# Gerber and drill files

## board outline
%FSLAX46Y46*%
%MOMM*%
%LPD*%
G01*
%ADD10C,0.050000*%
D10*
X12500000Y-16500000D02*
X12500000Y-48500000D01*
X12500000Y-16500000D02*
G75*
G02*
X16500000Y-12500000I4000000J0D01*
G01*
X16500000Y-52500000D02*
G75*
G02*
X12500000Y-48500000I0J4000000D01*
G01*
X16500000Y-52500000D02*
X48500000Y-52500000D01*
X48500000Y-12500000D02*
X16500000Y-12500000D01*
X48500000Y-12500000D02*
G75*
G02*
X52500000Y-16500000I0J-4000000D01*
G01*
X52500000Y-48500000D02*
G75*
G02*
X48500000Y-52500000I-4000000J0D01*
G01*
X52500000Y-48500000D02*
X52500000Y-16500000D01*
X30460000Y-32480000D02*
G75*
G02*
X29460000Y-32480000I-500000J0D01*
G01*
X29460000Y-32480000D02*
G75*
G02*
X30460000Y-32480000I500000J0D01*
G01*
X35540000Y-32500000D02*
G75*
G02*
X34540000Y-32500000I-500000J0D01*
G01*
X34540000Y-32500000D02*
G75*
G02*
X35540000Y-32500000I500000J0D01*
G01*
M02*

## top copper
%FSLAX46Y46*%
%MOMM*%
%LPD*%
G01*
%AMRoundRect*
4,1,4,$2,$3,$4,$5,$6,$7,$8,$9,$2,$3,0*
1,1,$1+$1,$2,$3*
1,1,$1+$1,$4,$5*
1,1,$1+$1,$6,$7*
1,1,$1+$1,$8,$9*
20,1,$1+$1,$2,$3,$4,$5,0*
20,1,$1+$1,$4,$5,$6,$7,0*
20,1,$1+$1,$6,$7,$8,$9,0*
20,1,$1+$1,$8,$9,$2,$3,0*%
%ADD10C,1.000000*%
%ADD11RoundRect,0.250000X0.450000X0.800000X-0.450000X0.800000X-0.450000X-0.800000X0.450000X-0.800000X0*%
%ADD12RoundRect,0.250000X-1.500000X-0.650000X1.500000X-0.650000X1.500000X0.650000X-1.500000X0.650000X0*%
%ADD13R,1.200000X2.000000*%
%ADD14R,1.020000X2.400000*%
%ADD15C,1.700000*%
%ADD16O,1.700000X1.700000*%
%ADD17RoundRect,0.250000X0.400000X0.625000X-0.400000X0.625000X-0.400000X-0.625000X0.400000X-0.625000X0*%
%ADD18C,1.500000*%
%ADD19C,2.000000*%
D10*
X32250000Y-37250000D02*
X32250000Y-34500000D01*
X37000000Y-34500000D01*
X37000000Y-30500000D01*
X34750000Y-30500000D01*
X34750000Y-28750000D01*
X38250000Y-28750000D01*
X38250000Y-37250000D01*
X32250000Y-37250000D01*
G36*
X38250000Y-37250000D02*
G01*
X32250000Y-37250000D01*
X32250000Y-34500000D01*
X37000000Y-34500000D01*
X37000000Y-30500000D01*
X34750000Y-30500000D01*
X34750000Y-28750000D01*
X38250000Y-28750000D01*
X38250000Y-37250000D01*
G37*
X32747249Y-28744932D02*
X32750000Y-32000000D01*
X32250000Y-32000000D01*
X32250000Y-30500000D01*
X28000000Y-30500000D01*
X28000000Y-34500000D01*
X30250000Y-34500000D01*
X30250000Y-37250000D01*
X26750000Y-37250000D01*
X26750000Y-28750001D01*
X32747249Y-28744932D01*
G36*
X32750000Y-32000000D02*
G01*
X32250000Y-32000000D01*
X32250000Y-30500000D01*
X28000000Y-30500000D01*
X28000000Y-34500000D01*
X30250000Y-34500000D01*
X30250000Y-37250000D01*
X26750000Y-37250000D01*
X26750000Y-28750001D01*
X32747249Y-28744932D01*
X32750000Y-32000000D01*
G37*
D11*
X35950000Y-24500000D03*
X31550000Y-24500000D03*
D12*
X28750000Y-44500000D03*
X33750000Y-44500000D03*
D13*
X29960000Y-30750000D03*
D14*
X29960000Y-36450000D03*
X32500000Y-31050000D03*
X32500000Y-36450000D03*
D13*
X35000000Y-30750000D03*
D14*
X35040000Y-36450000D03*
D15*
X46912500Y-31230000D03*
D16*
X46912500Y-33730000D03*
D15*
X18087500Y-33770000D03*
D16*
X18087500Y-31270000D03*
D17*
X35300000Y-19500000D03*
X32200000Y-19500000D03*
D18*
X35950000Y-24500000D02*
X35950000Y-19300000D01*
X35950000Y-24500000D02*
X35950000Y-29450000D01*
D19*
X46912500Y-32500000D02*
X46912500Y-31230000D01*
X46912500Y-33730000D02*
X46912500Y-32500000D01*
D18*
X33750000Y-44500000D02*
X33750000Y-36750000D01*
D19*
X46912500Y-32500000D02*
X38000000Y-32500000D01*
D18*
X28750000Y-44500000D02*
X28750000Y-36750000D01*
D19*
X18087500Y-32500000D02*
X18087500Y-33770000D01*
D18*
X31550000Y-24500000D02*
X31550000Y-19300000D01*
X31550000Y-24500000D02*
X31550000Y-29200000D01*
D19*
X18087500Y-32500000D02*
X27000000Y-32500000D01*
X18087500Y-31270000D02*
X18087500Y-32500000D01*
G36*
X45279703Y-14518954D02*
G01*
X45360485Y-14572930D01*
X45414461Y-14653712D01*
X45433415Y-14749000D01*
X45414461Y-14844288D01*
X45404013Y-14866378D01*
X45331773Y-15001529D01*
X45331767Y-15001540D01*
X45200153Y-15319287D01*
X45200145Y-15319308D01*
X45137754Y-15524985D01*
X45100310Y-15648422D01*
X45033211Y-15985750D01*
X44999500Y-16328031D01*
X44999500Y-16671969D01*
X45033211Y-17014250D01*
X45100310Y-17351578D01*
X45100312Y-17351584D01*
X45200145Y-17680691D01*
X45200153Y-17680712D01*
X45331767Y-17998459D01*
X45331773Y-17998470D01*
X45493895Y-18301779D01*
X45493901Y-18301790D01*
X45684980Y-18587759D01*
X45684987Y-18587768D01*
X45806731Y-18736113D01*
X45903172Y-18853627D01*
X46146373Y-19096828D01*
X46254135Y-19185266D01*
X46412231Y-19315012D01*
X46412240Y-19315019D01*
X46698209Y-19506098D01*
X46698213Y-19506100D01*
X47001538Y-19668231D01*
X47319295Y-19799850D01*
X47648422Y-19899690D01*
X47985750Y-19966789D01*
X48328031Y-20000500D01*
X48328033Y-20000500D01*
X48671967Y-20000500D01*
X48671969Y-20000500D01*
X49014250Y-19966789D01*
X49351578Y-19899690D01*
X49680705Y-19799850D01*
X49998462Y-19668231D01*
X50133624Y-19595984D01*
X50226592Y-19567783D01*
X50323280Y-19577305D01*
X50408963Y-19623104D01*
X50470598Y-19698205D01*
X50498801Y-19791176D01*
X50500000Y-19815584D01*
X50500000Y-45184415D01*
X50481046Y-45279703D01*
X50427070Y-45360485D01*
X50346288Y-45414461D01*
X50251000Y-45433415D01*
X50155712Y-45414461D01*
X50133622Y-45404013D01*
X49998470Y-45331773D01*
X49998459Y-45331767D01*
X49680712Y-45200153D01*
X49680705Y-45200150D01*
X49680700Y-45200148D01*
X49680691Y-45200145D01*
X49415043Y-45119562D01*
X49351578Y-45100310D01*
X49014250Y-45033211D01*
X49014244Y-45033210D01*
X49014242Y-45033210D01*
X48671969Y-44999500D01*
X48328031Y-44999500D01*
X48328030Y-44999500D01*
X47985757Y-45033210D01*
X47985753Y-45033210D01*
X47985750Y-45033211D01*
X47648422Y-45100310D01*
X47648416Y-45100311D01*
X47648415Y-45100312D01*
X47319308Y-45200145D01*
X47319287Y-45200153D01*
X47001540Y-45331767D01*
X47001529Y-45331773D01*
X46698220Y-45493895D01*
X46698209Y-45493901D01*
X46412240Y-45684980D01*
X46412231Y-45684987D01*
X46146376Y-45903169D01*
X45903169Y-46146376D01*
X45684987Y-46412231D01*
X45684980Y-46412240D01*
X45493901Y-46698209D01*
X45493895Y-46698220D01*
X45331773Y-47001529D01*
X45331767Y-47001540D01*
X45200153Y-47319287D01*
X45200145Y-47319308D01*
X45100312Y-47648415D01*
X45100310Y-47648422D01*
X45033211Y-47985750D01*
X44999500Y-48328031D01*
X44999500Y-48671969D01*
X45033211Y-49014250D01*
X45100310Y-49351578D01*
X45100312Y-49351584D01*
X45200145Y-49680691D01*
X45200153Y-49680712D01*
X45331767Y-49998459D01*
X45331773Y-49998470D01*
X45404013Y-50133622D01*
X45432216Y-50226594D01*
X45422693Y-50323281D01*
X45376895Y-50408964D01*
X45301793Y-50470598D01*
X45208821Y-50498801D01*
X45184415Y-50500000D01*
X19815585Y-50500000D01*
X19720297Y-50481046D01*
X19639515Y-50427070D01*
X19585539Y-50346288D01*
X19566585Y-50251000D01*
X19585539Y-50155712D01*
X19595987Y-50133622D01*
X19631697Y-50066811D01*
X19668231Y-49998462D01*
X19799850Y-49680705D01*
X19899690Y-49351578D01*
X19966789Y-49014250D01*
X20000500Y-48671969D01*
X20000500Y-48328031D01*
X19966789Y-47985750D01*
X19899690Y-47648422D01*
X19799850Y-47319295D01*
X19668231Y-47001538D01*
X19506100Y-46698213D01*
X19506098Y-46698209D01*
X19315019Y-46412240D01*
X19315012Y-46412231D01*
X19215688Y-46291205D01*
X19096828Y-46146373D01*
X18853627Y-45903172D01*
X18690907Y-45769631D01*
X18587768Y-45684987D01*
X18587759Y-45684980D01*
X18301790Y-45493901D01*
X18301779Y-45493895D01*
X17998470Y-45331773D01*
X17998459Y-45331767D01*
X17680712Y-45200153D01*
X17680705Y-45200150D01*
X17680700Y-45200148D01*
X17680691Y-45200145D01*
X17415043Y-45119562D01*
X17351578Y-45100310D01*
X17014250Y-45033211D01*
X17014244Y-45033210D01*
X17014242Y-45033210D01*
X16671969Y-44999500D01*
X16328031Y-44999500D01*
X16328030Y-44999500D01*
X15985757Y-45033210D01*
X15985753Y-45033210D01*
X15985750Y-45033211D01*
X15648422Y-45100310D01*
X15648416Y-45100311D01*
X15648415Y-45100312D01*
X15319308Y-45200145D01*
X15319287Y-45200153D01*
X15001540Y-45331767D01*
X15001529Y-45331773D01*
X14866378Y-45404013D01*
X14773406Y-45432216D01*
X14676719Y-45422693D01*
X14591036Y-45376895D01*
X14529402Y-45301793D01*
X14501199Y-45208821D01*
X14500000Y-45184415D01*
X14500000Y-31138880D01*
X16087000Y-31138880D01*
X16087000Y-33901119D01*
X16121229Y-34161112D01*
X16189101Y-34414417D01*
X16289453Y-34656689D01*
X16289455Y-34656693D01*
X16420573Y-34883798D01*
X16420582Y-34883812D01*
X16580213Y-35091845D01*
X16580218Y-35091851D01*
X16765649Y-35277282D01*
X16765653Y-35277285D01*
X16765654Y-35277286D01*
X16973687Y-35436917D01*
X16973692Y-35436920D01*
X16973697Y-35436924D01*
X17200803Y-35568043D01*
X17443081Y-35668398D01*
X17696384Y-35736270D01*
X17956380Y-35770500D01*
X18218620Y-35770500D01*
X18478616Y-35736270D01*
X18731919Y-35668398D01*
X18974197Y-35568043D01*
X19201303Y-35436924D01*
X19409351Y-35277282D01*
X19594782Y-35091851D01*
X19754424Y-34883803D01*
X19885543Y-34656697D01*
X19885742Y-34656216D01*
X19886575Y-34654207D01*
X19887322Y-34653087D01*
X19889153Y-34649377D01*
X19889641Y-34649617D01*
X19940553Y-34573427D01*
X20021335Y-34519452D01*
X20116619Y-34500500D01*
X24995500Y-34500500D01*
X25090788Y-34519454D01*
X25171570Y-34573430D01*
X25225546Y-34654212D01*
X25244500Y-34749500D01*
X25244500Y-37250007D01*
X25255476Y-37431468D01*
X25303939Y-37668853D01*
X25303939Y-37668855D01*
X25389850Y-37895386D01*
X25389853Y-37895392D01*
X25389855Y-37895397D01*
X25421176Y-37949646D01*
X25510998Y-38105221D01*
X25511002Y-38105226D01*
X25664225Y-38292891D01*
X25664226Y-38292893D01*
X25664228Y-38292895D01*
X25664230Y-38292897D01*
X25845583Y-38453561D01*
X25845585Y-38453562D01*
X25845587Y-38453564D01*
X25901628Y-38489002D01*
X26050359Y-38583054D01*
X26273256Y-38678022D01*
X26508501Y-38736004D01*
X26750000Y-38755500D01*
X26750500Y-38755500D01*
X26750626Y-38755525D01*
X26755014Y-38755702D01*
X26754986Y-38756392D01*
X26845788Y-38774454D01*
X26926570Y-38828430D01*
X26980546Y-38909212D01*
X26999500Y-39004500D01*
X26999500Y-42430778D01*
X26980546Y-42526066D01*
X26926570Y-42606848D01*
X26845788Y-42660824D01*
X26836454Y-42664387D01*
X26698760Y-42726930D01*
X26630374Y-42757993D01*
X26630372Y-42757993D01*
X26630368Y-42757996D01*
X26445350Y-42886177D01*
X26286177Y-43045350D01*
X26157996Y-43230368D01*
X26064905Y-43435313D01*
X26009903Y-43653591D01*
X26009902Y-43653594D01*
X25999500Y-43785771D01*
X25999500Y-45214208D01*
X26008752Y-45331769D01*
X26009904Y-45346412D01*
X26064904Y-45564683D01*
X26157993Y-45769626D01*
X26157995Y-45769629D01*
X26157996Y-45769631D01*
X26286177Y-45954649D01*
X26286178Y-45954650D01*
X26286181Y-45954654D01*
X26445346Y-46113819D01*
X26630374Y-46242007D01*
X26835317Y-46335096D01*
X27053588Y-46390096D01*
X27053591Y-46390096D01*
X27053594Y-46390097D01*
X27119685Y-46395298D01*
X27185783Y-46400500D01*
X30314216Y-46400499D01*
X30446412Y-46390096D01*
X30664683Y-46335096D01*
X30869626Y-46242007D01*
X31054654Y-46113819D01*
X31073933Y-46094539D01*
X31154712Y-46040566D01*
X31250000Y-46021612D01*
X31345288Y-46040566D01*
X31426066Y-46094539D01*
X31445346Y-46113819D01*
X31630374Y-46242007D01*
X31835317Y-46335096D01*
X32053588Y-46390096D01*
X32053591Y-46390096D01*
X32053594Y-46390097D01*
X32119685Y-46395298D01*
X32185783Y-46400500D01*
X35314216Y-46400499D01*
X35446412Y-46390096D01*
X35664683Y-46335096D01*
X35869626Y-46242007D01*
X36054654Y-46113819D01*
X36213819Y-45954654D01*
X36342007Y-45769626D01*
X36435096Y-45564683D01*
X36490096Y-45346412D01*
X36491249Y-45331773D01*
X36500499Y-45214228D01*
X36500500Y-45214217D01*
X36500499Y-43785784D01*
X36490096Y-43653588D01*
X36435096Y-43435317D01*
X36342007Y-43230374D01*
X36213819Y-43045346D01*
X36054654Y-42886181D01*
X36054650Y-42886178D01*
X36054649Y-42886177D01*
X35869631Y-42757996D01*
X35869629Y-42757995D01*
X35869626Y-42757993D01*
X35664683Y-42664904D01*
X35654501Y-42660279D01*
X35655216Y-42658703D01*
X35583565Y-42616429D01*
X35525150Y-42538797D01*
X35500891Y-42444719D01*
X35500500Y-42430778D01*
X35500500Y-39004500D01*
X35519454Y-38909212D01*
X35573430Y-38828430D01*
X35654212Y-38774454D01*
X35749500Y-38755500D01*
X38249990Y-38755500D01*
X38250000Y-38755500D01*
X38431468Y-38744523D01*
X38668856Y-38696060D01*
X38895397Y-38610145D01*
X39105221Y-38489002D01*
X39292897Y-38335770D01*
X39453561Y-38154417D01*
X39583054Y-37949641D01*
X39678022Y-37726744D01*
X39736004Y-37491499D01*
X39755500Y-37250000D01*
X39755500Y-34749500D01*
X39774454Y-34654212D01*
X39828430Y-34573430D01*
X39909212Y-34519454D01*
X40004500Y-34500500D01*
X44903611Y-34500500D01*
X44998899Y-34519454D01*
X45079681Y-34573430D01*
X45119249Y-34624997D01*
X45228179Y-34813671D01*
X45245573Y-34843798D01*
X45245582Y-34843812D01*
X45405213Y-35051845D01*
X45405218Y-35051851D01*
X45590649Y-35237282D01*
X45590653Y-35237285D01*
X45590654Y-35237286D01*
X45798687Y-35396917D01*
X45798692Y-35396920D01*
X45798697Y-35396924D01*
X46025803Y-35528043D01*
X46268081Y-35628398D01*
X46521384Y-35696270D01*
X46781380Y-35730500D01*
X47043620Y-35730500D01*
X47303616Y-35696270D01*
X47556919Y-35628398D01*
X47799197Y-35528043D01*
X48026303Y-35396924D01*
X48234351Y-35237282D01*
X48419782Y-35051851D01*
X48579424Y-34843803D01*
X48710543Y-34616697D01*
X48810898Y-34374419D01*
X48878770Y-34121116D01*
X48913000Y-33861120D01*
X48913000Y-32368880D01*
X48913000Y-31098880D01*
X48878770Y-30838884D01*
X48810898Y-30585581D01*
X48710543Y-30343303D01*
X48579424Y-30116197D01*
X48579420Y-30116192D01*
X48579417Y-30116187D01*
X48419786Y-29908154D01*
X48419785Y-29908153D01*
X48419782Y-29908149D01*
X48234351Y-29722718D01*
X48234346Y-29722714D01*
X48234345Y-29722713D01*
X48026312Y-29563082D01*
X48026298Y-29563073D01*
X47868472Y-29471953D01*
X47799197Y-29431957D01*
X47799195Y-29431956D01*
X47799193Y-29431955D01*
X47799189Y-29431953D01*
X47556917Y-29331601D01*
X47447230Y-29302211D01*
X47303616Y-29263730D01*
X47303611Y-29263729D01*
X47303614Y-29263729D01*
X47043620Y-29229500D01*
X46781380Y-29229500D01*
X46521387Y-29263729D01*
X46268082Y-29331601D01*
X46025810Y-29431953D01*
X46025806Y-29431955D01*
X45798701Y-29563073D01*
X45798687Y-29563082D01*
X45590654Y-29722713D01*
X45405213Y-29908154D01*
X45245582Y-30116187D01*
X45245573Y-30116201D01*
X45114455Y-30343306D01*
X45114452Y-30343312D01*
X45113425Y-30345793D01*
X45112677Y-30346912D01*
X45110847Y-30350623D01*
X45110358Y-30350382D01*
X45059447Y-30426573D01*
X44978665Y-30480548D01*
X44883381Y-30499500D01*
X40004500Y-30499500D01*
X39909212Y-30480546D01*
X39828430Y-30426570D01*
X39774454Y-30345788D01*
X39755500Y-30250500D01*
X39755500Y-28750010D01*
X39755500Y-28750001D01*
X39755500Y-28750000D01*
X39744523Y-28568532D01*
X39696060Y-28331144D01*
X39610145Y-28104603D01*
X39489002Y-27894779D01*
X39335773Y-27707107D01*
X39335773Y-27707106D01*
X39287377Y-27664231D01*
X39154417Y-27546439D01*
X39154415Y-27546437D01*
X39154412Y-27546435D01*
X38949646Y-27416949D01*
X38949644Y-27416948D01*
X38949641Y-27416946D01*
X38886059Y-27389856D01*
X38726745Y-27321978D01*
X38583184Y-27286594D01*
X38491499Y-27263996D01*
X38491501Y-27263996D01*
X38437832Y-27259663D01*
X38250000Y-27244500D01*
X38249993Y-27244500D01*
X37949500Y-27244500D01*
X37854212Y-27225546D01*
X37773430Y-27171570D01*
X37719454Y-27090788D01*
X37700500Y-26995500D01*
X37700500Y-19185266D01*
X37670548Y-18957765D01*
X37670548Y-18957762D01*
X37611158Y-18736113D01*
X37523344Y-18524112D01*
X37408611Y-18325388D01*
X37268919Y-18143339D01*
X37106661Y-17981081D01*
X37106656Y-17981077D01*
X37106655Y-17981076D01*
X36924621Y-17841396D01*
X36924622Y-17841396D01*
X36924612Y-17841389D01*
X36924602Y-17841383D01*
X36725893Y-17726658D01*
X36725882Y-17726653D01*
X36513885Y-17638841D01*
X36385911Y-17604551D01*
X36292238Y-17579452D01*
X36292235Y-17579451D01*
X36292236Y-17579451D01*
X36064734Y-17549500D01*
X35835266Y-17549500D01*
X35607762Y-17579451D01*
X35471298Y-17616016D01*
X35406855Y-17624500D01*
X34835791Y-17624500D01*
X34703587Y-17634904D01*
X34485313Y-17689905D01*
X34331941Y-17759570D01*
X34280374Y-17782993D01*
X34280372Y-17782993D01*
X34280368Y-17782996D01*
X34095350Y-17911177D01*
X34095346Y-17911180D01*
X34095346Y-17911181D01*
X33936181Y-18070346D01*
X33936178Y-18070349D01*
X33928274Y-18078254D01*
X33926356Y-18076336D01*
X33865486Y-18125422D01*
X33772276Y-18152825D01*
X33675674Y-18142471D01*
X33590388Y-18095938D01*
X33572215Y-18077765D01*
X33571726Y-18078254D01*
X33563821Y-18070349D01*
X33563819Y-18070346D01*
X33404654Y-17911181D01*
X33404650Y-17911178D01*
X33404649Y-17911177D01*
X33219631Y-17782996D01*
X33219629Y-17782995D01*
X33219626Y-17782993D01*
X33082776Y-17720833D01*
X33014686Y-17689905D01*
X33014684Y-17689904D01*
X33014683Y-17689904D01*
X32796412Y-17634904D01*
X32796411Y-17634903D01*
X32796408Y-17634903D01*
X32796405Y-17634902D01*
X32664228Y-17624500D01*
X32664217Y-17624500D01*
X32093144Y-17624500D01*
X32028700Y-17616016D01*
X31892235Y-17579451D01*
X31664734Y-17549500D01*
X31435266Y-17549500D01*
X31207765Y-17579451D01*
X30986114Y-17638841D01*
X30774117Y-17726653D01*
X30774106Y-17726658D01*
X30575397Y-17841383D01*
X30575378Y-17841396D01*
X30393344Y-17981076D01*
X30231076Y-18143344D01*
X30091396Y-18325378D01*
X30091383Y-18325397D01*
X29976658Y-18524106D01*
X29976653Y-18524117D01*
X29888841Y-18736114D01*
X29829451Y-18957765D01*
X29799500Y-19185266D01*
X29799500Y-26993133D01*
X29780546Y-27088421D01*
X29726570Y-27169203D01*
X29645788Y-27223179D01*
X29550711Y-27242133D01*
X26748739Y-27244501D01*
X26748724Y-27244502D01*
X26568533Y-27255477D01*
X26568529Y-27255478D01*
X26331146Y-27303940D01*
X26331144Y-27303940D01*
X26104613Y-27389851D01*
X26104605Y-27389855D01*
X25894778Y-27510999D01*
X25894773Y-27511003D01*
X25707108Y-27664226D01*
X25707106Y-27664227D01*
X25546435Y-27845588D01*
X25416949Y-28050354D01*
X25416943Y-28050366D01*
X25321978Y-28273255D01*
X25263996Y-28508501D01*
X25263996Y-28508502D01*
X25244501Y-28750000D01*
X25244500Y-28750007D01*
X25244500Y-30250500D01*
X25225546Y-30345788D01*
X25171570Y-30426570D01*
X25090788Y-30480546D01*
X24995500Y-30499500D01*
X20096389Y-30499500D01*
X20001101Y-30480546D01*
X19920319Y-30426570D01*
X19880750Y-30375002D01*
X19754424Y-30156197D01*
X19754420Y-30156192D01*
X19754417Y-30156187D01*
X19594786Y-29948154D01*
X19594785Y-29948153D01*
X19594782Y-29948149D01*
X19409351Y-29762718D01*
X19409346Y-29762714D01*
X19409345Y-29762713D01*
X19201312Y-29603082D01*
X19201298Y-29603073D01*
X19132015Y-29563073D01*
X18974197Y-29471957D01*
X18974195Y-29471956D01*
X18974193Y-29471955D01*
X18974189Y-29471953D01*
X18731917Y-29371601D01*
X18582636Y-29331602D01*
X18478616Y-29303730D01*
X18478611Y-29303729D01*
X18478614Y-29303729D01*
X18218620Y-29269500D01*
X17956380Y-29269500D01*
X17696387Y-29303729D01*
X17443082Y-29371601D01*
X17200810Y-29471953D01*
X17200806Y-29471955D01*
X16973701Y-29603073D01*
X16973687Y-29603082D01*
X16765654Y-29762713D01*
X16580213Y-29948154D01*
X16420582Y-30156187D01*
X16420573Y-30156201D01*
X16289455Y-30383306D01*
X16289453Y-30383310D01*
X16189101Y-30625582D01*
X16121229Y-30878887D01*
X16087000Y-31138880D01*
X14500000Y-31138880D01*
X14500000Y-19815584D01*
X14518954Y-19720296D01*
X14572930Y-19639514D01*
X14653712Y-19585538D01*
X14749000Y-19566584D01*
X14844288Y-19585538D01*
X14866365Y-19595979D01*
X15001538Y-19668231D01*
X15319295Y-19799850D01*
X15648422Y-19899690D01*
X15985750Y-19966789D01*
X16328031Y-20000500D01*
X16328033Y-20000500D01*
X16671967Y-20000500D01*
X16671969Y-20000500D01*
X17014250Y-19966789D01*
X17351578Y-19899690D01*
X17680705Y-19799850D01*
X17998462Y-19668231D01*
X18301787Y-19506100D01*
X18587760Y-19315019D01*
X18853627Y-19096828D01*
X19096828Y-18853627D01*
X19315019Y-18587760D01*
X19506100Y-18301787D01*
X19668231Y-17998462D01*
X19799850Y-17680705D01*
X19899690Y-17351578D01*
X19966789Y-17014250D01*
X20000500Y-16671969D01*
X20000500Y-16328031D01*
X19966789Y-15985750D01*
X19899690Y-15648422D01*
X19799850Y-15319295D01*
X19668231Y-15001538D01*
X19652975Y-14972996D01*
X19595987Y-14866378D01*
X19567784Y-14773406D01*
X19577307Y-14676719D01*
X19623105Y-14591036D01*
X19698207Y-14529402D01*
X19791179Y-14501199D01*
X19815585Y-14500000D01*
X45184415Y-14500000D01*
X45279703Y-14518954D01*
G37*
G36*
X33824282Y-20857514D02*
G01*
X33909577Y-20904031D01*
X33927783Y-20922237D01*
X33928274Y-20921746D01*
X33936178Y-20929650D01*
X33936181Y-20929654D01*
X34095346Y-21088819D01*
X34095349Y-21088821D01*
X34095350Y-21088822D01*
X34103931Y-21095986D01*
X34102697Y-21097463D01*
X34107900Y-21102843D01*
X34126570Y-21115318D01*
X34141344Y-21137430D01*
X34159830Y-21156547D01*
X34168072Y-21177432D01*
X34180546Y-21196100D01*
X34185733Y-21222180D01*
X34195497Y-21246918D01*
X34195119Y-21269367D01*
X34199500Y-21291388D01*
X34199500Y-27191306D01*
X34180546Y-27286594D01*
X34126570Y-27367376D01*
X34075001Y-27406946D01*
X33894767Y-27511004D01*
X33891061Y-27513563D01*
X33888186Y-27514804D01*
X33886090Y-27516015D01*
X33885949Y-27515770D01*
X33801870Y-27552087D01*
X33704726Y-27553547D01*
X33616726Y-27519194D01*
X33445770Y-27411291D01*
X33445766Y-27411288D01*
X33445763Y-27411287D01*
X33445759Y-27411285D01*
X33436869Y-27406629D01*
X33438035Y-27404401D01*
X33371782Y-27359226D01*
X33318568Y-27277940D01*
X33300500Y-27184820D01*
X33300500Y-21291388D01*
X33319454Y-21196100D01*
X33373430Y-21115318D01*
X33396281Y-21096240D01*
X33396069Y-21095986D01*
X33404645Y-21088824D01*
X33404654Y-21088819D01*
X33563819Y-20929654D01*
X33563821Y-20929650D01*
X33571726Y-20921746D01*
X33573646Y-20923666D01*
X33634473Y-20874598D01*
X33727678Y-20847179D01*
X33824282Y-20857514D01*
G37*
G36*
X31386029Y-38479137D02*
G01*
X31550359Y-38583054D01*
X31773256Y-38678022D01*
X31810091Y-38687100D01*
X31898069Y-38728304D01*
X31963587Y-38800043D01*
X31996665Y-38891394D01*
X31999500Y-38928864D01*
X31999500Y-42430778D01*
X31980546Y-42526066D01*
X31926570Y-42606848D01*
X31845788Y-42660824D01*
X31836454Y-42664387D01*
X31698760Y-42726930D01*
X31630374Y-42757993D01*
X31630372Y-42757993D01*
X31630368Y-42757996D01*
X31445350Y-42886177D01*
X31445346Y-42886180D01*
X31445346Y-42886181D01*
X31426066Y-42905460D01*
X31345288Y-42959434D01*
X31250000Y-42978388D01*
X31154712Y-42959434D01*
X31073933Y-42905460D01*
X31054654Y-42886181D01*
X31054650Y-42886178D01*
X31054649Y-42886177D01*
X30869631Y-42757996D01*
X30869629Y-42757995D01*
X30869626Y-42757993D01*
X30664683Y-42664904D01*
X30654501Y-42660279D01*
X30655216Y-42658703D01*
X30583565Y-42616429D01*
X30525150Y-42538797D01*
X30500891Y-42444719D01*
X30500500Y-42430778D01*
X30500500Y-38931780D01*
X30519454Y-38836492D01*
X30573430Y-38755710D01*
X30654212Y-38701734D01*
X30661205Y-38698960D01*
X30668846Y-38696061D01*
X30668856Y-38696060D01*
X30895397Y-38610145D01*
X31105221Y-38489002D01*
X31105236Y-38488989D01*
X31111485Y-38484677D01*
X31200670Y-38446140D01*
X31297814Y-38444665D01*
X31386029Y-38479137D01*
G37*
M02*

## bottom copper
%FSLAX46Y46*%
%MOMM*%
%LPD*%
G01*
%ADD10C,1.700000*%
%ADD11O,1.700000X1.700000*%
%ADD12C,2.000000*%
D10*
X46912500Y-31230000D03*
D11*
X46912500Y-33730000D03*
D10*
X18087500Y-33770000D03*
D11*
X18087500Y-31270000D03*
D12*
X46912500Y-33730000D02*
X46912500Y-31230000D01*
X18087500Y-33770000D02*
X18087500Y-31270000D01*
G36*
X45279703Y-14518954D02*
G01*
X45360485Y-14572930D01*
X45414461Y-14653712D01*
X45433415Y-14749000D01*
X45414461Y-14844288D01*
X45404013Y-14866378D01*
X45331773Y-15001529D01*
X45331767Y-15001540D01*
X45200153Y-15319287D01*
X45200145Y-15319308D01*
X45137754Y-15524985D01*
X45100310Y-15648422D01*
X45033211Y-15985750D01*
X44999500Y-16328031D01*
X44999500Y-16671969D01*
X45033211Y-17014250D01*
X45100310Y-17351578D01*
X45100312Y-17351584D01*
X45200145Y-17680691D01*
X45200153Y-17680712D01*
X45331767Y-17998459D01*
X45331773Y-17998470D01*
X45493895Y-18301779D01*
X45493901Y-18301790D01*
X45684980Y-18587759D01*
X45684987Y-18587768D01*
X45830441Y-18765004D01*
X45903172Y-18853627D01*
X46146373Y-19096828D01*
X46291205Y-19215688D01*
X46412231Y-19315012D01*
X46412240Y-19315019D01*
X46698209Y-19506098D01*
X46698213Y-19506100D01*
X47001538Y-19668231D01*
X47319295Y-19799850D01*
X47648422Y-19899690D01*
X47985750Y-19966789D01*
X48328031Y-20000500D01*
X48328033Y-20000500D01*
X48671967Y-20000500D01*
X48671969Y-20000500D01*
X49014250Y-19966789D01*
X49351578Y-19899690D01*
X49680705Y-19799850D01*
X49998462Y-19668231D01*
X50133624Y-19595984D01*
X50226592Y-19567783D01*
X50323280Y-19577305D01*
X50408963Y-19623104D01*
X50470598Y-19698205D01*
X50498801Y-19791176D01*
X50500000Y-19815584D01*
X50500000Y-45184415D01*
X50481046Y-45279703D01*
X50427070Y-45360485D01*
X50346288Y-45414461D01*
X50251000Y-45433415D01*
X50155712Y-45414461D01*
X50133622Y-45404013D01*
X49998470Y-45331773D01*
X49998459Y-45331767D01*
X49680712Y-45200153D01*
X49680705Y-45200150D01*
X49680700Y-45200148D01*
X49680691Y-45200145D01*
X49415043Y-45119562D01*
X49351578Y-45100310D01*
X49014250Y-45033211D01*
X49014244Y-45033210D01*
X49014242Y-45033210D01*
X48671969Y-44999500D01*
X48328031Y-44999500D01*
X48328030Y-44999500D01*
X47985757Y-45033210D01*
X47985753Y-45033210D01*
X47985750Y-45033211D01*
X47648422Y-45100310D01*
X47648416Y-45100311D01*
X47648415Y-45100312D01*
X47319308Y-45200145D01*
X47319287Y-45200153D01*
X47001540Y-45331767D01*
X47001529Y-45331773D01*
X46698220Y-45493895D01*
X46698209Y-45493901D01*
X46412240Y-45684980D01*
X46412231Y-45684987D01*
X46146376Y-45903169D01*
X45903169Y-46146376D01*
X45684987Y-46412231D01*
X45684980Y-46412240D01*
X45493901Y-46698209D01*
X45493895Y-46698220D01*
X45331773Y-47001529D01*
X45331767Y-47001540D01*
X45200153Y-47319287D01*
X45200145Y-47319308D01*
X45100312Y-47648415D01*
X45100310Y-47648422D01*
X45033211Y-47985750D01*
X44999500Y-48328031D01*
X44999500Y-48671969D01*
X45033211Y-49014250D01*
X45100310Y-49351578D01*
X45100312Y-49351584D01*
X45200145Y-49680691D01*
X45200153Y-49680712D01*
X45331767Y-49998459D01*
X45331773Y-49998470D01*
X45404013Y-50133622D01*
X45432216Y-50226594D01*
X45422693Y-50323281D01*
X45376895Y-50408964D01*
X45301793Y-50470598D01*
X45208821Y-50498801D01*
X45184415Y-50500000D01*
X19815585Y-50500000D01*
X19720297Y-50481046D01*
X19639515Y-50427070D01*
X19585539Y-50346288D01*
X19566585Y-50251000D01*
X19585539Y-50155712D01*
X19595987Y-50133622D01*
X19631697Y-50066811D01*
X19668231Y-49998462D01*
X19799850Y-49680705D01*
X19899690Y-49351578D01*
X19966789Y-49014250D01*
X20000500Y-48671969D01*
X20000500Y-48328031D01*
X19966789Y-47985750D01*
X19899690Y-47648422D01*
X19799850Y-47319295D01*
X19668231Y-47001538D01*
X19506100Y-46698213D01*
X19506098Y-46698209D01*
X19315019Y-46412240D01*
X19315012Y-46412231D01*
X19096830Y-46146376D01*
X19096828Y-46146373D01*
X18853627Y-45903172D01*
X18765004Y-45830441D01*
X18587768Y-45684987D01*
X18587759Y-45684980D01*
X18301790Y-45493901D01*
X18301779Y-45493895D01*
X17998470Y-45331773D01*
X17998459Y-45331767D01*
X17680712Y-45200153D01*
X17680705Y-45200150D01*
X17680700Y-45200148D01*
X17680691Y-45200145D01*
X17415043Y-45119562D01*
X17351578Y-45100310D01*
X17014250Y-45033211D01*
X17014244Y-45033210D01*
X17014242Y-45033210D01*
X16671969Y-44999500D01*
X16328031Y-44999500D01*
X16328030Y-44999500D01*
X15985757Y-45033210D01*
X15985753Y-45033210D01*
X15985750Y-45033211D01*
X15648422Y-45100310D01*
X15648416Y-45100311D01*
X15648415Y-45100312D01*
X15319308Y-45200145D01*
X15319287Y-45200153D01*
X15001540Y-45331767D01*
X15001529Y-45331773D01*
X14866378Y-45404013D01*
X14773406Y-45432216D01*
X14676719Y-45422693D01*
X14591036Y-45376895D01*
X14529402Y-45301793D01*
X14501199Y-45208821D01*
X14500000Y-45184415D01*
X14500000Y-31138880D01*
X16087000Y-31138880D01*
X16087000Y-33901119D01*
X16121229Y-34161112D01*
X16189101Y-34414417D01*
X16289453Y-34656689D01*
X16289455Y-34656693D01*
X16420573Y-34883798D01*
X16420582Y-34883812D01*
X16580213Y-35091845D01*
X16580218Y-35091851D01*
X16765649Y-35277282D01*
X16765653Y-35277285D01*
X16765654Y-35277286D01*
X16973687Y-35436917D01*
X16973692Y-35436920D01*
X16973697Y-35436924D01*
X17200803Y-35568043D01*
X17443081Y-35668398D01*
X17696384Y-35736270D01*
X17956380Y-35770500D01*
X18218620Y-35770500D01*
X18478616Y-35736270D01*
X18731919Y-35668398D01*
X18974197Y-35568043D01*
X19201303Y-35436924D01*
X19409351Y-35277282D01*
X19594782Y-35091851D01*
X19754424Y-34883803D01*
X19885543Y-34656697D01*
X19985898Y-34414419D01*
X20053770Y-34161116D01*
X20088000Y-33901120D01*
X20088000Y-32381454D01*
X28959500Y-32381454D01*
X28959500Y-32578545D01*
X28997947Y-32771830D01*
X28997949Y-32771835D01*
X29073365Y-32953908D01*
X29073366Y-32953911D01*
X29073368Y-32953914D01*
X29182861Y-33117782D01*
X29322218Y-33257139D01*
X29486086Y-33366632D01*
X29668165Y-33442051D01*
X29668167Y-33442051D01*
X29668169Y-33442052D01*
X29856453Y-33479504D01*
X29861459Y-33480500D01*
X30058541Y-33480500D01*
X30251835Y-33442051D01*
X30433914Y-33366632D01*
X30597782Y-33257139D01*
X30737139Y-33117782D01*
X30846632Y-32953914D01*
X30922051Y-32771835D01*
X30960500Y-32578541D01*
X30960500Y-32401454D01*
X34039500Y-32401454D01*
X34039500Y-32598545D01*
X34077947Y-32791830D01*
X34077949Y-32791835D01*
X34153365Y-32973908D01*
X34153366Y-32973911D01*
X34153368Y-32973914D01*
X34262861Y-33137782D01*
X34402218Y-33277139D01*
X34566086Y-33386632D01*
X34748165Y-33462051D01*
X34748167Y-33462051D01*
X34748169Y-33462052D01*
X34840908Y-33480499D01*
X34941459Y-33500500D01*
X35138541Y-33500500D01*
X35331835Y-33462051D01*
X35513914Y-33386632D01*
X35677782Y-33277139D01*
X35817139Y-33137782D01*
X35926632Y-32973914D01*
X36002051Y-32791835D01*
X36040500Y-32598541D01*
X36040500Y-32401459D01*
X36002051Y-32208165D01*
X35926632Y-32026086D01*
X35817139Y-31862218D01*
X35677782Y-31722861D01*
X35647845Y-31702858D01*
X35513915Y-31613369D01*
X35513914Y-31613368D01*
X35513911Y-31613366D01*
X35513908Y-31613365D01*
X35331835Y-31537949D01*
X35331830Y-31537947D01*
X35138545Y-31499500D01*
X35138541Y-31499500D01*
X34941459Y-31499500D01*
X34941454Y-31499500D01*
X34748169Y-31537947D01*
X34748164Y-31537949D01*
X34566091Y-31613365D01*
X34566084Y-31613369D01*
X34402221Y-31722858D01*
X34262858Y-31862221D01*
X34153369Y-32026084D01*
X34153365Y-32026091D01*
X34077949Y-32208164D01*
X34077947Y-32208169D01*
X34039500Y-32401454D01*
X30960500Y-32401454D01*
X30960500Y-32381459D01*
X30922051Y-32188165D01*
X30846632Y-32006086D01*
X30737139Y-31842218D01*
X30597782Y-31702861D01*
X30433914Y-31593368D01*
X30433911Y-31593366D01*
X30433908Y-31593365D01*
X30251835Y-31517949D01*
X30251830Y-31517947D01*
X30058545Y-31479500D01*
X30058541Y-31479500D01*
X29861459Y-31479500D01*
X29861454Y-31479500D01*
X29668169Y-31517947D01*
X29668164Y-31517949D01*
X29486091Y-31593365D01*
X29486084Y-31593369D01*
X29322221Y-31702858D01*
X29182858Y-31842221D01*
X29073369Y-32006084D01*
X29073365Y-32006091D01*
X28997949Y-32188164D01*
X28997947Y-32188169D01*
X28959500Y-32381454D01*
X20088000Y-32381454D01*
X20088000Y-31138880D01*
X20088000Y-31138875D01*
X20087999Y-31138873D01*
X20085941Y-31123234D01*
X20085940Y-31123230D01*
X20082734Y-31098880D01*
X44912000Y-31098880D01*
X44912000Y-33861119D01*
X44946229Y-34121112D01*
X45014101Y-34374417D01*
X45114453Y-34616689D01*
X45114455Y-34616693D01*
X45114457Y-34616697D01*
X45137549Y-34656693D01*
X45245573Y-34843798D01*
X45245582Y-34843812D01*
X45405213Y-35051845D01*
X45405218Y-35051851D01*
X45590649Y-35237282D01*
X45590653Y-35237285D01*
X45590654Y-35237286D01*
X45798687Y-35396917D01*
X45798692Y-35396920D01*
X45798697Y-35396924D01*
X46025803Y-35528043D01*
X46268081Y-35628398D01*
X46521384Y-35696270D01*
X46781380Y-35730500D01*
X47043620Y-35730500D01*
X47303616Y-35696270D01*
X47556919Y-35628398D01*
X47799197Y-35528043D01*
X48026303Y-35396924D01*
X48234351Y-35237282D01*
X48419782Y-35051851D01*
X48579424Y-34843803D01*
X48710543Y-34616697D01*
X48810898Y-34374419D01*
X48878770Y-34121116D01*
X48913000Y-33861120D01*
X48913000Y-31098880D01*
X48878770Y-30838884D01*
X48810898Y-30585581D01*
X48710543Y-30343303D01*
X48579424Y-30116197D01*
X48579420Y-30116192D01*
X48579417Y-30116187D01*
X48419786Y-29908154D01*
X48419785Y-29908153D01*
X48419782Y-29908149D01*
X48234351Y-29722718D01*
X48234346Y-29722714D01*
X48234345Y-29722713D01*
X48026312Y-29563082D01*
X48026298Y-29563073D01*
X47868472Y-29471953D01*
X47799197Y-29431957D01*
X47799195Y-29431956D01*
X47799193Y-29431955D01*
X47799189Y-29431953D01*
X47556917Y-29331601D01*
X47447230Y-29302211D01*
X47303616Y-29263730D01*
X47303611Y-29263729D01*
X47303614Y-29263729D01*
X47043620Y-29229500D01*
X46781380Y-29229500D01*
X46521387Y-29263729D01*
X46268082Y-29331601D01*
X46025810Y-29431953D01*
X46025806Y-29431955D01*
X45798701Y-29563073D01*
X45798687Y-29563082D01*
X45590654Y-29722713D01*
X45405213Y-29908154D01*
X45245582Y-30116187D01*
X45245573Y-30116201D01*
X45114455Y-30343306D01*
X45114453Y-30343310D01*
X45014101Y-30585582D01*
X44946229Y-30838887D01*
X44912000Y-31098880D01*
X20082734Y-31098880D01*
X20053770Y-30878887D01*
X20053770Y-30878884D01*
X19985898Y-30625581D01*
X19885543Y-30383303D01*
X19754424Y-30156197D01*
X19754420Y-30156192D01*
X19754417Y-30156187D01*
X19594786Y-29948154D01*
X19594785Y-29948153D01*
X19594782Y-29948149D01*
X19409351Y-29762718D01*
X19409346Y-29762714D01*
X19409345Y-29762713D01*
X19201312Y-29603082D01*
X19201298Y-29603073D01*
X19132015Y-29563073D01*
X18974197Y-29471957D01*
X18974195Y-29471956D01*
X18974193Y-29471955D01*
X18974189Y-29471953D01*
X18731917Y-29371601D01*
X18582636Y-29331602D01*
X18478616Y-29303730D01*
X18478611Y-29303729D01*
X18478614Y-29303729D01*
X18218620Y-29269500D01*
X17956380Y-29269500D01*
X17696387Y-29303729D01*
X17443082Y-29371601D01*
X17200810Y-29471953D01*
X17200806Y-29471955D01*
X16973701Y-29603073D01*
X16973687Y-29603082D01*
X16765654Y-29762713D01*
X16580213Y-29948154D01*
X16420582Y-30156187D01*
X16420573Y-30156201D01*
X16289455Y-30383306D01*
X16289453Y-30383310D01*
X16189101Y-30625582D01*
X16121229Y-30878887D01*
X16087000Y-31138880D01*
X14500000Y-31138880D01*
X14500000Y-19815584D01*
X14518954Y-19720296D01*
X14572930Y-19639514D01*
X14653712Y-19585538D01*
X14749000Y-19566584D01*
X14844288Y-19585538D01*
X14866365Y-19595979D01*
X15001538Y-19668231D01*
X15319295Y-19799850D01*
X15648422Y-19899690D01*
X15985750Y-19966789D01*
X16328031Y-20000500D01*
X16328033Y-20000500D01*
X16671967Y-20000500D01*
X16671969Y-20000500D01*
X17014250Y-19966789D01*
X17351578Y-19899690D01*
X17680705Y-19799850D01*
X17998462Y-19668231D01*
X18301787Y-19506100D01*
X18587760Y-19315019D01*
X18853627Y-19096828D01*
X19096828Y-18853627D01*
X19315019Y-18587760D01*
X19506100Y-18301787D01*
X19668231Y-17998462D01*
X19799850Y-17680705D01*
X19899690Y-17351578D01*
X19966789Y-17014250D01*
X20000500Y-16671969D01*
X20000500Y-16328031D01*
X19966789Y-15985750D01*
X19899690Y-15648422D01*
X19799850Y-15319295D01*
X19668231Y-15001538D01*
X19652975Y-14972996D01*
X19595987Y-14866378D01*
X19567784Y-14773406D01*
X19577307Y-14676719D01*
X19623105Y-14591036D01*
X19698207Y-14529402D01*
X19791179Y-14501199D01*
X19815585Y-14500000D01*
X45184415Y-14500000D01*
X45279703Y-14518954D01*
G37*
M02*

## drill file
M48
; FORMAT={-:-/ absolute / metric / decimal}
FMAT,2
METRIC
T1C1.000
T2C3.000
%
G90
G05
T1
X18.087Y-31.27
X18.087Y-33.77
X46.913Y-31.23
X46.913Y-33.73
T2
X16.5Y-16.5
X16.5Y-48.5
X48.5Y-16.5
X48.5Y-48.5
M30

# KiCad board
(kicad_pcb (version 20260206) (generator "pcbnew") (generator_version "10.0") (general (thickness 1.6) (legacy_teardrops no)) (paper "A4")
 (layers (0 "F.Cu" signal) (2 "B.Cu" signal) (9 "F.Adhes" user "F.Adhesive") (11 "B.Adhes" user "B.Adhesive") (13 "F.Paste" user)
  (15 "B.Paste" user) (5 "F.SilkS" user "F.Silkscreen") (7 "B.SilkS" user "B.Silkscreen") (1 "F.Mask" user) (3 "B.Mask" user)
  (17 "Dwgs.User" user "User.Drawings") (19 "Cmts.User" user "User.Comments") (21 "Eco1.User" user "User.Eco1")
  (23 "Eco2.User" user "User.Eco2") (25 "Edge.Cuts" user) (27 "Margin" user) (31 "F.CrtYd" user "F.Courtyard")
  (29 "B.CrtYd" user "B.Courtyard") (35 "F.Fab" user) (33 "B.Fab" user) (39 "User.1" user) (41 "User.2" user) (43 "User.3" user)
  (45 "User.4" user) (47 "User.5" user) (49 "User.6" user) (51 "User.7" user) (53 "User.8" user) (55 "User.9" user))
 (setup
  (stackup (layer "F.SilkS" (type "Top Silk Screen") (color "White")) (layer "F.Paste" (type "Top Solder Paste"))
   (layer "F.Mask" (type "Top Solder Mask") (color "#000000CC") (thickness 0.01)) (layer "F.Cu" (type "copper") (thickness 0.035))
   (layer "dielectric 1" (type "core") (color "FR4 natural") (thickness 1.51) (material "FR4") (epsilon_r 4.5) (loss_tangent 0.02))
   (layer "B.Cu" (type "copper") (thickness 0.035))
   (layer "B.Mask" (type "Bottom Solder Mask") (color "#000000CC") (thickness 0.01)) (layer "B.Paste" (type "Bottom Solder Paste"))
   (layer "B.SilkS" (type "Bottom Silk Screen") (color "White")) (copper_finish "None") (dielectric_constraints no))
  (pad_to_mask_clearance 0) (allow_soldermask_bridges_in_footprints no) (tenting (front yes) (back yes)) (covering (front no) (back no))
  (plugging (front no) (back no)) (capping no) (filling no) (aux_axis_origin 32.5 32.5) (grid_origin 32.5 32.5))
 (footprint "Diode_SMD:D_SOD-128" (layer "F.Cu") (at 33.75 24.5 180)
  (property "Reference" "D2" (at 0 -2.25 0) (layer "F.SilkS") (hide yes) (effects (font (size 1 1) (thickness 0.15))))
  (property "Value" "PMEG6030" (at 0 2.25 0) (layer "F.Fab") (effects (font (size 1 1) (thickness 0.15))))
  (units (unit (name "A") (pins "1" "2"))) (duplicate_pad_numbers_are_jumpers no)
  (pad "1" smd roundrect (at -2.2 0 180) (size 1.4 2.1) (layers "F.Cu" "F.Mask" "F.Paste") (roundrect_rratio 0.1785714286)
   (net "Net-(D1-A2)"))
  (pad "2" smd roundrect (at 2.2 0 180) (size 1.4 2.1) (layers "F.Cu" "F.Mask" "F.Paste") (roundrect_rratio 0.1785714286)
   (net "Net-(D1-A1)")))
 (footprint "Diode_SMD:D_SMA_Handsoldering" (layer "F.Cu") (at 31.25 44.5)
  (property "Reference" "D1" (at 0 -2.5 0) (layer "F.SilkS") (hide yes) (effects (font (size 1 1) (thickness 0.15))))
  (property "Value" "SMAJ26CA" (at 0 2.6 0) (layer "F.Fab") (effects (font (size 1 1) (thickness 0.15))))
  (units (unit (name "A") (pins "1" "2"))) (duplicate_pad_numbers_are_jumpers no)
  (pad "1" smd roundrect (at -2.5 0) (size 3.5 1.8) (layers "F.Cu" "F.Mask" "F.Paste") (roundrect_rratio 0.1388888889) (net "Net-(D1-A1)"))
  (pad "2" smd roundrect (at 2.5 0) (size 3.5 1.8) (layers "F.Cu" "F.Mask" "F.Paste") (roundrect_rratio 0.1388888889) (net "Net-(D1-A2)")))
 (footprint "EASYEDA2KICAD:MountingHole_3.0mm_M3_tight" (layer "F.Cu") (at 16.5 16.5 90)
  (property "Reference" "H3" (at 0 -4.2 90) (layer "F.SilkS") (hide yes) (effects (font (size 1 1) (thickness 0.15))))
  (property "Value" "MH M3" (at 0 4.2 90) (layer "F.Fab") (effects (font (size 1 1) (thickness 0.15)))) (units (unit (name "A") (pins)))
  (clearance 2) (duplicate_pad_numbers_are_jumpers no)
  (pad "" np_thru_hole circle (at 0 0 90) (size 3 3) (drill 3) (layers "*.Cu" "*.Mask")))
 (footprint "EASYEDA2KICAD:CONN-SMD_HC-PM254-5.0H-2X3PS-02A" (layer "F.Cu") (at 32.5 33.75)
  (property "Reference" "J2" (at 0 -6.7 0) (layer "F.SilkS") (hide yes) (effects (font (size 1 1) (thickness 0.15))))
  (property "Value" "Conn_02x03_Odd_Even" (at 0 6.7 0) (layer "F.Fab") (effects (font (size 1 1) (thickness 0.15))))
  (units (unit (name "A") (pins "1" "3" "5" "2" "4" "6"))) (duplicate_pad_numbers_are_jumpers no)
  (fp_circle (center -2.54 -1.27) (end -2.04 -1.27) (stroke (width 0.05) (type default)) (fill no) (layer "Edge.Cuts"))
  (fp_circle (center 2.54 -1.25) (end 3.04 -1.25) (stroke (width 0.05) (type default)) (fill no) (layer "Edge.Cuts"))
  (pad "1" smd rect (at -2.54 -3 180) (size 1.2 2) (layers "F.Cu" "F.Mask" "F.Paste") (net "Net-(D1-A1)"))
  (pad "2" smd rect (at -2.54 2.7) (size 1.02 2.4) (layers "F.Cu" "F.Mask" "F.Paste") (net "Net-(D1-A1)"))
  (pad "3" smd rect (at 0 -2.7) (size 1.02 2.4) (layers "F.Cu" "F.Mask" "F.Paste") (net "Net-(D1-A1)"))
  (pad "4" smd rect (at 0 2.7) (size 1.02 2.4) (layers "F.Cu" "F.Mask" "F.Paste") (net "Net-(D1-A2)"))
  (pad "5" smd rect (at 2.5 -3 180) (size 1.2 2) (layers "F.Cu" "F.Mask" "F.Paste") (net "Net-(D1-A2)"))
  (pad "6" smd rect (at 2.54 2.7) (size 1.02 2.4) (layers "F.Cu" "F.Mask" "F.Paste") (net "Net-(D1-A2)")))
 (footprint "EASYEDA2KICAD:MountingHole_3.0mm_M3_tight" (layer "F.Cu") (at 16.5 48.5 90)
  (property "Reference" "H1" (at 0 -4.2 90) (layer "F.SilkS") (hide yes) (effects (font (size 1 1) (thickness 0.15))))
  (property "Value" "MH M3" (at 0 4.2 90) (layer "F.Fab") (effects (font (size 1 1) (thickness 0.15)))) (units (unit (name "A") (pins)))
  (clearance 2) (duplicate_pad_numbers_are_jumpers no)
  (pad "" np_thru_hole circle (at 0 0 90) (size 3 3) (drill 3) (layers "*.Cu" "*.Mask")))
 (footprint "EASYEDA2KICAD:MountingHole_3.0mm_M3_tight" (layer "F.Cu") (at 48.5 16.5 90)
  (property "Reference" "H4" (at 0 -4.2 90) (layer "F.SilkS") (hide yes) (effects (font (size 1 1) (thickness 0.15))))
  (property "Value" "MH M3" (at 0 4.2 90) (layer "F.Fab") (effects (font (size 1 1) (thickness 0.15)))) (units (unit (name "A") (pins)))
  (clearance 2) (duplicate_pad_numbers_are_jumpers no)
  (pad "" np_thru_hole circle (at 0 0 90) (size 3 3) (drill 3) (layers "*.Cu" "*.Mask")))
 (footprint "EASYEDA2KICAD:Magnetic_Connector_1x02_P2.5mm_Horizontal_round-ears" (layer "F.Cu") (at 47.0125 32.5)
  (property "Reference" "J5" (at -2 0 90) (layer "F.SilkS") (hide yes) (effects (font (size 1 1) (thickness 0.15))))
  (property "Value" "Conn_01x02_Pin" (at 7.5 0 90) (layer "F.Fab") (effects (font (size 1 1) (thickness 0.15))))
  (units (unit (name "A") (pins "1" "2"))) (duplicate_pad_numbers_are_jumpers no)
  (pad "1" thru_hole circle (at -0.1 -1.27) (size 1.7 1.7) (drill 1) (layers "*.Cu" "*.Mask") (remove_unused_layers no) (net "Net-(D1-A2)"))
  (pad "2" thru_hole oval (at -0.1 1.23) (size 1.7 1.7) (drill 1) (layers "*.Cu" "*.Mask") (remove_unused_layers no) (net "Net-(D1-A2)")))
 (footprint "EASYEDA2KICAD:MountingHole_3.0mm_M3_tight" (layer "F.Cu") (at 48.5 48.5 90)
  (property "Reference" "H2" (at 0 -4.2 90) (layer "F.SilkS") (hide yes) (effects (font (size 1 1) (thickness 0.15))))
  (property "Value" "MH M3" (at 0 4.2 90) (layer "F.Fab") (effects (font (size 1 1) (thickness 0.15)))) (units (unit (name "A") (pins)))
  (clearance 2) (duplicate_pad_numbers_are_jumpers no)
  (pad "" np_thru_hole circle (at 0 0 90) (size 3 3) (drill 3) (layers "*.Cu" "*.Mask")))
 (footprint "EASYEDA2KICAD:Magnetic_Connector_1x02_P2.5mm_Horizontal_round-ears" (layer "F.Cu") (at 17.9875 32.5 180)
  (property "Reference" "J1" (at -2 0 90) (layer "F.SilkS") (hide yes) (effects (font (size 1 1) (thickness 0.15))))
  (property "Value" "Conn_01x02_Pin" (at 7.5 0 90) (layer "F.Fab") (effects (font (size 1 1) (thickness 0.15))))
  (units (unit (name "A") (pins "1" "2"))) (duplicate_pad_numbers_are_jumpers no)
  (pad "1" thru_hole circle (at -0.1 -1.27 180) (size 1.7 1.7) (drill 1) (layers "*.Cu" "*.Mask") (remove_unused_layers no)
   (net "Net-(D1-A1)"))
  (pad "2" thru_hole oval (at -0.1 1.23 180) (size 1.7 1.7) (drill 1) (layers "*.Cu" "*.Mask") (remove_unused_layers no) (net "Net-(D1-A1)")))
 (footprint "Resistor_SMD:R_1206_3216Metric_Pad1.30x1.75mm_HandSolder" (layer "F.Cu") (at 33.75 19.5 180)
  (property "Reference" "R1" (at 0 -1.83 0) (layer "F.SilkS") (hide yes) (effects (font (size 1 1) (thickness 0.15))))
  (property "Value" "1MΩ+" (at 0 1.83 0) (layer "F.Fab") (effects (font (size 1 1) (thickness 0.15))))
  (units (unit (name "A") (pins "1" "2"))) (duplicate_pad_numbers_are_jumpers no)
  (pad "1" smd roundrect (at -1.55 0 180) (size 1.3 1.75) (layers "F.Cu" "F.Mask" "F.Paste") (roundrect_rratio 0.192308) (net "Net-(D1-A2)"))
  (pad "2" smd roundrect (at 1.55 0 180) (size 1.3 1.75) (layers "F.Cu" "F.Mask" "F.Paste") (roundrect_rratio 0.192308) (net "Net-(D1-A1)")))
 (gr_poly
  (pts (xy 32.25 37.25) (xy 32.25 34.5) (xy 37 34.5) (xy 37 30.5) (xy 34.75 30.5) (xy 34.75 28.75) (xy 38.25 28.75) (xy 38.25 37.25))
  (stroke (width 1) (type solid)) (fill yes) (layer "F.Cu") (net "Net-(D1-A2)"))
 (gr_poly
  (pts (xy 32.747249 28.744932) (xy 32.75 32) (xy 32.25 32) (xy 32.25 30.5) (xy 28 30.5) (xy 28 34.5) (xy 30.25 34.5) (xy 30.25 37.25)
   (xy 26.75 37.25) (xy 26.75 28.750001))
  (stroke (width 1) (type solid)) (fill yes) (layer "F.Cu") (net "Net-(D1-A1)"))
 (gr_line (start 12.5 16.5) (end 12.5 48.5) (stroke (width 0.05) (type default)) (layer "Edge.Cuts"))
 (gr_arc (start 12.5 16.5) (mid 13.671573 13.671573) (end 16.5 12.5) (stroke (width 0.05) (type default)) (layer "Edge.Cuts"))
 (gr_arc (start 16.5 52.5) (mid 13.671573 51.328427) (end 12.5 48.5) (stroke (width 0.05) (type default)) (layer "Edge.Cuts"))
 (gr_line (start 16.5 52.5) (end 48.5 52.5) (stroke (width 0.05) (type default)) (layer "Edge.Cuts"))
 (gr_line (start 48.5 12.5) (end 16.5 12.5) (stroke (width 0.05) (type default)) (layer "Edge.Cuts"))
 (gr_arc (start 48.5 12.5) (mid 51.328427 13.671573) (end 52.5 16.5) (stroke (width 0.05) (type default)) (layer "Edge.Cuts"))
 (gr_arc (start 52.5 48.5) (mid 51.328427 51.328427) (end 48.5 52.5) (stroke (width 0.05) (type default)) (layer "Edge.Cuts"))
 (gr_line (start 52.5 48.5) (end 52.5 16.5) (stroke (width 0.05) (type default)) (layer "Edge.Cuts"))
 (segment (start 35.95 24.5) (end 35.95 19.3) (width 1.5) (layer "F.Cu") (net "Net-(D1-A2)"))
 (segment (start 35.95 24.5) (end 35.95 29.45) (width 1.5) (layer "F.Cu") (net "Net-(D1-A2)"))
 (segment (start 46.9125 32.5) (end 46.9125 31.23) (width 2) (layer "F.Cu") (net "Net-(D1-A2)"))
 (segment (start 46.9125 33.73) (end 46.9125 32.5) (width 2) (layer "F.Cu") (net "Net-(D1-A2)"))
 (segment (start 33.75 44.5) (end 33.75 36.75) (width 1.5) (layer "F.Cu") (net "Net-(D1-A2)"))
 (segment (start 46.9125 32.5) (end 38 32.5) (width 2) (layer "F.Cu") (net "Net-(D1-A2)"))
 (segment (start 46.9125 33.73) (end 46.9125 31.23) (width 2) (layer "B.Cu") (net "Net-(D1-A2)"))
 (segment (start 28.75 44.5) (end 28.75 36.75) (width 1.5) (layer "F.Cu") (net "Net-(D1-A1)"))
 (segment (start 18.0875 32.5) (end 18.0875 33.77) (width 2) (layer "F.Cu") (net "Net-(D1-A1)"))
 (segment (start 31.55 24.5) (end 31.55 19.3) (width 1.5) (layer "F.Cu") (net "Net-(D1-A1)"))
 (segment (start 31.55 24.5) (end 31.55 29.2) (width 1.5) (layer "F.Cu") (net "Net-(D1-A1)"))
 (segment (start 18.0875 32.5) (end 27 32.5) (width 2) (layer "F.Cu") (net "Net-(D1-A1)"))
 (segment (start 18.0875 31.27) (end 18.0875 32.5) (width 2) (layer "F.Cu") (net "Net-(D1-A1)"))
 (segment (start 18.0875 33.77) (end 18.0875 31.27) (width 2) (layer "B.Cu") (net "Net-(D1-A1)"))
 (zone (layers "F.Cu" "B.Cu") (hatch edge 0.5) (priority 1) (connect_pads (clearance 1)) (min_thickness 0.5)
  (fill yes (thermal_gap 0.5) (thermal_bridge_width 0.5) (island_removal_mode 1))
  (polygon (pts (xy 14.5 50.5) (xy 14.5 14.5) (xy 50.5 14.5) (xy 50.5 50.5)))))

